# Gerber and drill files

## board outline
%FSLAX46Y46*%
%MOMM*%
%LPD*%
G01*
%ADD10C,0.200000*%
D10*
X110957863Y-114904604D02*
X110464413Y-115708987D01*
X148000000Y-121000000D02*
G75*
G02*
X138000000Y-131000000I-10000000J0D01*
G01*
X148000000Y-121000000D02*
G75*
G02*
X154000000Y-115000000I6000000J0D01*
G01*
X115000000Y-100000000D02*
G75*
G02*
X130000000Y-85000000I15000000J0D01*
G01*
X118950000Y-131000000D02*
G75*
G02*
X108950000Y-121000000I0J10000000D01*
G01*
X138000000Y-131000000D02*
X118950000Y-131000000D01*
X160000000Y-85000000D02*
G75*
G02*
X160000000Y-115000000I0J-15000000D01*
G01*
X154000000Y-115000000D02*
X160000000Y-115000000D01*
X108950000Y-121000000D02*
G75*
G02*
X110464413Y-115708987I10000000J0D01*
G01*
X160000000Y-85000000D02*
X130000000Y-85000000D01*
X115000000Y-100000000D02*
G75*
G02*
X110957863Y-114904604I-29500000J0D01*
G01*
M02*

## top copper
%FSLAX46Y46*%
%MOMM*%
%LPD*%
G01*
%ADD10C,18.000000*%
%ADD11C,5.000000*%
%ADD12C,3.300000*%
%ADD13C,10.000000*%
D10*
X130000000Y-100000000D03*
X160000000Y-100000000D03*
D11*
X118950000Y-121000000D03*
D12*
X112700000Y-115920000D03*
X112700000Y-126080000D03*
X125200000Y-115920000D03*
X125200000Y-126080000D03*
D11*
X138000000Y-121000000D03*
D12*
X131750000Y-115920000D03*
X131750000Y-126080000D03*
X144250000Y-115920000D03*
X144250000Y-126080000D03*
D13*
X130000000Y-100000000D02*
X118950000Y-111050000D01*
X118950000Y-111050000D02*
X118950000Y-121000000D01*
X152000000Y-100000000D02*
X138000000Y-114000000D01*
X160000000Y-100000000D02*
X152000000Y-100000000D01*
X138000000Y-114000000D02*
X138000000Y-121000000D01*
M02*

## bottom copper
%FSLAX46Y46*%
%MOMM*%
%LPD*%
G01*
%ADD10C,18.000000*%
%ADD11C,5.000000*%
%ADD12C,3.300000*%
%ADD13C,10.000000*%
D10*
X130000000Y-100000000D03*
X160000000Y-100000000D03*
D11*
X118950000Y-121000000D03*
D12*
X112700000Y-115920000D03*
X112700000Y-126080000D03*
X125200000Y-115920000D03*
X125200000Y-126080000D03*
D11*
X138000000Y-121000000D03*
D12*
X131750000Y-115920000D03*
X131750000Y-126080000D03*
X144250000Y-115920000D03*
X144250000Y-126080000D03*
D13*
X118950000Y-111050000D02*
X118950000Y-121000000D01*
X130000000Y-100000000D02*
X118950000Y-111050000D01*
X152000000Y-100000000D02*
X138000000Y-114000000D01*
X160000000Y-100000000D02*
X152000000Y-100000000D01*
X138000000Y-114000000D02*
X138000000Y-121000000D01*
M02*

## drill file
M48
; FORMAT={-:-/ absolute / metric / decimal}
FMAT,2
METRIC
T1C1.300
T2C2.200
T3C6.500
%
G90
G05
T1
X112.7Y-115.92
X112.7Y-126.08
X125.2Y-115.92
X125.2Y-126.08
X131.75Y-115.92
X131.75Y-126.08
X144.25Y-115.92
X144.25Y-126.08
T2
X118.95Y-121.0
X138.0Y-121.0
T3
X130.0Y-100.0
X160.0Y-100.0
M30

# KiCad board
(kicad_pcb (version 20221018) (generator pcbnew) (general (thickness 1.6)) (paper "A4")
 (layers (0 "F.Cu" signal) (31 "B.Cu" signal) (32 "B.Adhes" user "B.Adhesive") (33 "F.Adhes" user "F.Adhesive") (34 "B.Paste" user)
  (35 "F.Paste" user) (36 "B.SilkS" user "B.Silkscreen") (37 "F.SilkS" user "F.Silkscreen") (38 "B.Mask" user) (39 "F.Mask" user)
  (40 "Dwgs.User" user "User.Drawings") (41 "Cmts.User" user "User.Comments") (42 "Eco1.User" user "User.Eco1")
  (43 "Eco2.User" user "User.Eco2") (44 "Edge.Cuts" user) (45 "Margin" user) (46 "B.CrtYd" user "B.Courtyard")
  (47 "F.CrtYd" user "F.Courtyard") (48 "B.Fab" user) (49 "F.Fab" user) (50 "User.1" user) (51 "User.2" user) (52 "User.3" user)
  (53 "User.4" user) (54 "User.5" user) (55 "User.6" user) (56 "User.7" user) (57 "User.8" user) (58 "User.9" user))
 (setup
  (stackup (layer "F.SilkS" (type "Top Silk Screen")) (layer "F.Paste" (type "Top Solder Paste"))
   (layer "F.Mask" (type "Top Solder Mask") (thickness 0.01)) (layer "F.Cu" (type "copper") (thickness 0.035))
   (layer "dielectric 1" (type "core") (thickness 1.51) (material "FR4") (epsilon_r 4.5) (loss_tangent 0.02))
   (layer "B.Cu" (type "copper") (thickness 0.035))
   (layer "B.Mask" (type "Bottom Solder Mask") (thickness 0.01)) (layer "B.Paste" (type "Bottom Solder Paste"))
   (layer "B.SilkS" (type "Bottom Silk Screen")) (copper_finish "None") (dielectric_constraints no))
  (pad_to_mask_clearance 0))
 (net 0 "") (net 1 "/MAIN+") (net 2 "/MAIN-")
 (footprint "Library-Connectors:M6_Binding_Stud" (layer "F.Cu") (at 130 100)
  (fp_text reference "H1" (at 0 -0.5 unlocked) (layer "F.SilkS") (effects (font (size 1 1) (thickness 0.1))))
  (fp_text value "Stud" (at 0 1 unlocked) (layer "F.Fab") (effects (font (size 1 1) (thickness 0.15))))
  (pad "1" thru_hole circle (at 0 0) (size 18 18) (drill 6.5) (layers "*.Cu" "*.Mask") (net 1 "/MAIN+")))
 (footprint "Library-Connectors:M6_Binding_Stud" (layer "F.Cu") (at 160 100)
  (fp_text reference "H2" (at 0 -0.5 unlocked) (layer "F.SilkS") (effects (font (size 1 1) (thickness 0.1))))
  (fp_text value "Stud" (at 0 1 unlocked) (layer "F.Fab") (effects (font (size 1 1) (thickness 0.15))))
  (pad "1" thru_hole circle (at 0 0) (size 18 18) (drill 6.5) (layers "*.Cu" "*.Mask") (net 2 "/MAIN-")))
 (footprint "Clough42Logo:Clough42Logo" (layer "F.Cu") (at 145.5 87.5)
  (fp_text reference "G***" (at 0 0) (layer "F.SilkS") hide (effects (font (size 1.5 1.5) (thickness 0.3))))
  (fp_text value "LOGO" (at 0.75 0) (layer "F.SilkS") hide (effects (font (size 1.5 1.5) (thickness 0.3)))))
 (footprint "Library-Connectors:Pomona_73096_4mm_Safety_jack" (layer "F.Cu") (at 118.95 121)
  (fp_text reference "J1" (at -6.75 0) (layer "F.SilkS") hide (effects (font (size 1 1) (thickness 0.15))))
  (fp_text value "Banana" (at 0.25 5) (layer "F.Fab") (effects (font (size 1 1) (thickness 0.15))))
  (pad "1" thru_hole circle (at 0 0) (size 5 5) (drill 2.2) (layers "*.Cu" "*.Mask") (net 1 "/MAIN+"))
  (pad "2" thru_hole circle (at -6.25 -5.08) (size 3.3 3.3) (drill 1.3) (layers "*.Cu" "*.Mask"))
  (pad "2" thru_hole circle (at -6.25 5.08) (size 3.3 3.3) (drill 1.3) (layers "*.Cu" "*.Mask"))
  (pad "2" thru_hole circle (at 6.25 -5.08) (size 3.3 3.3) (drill 1.3) (layers "*.Cu" "*.Mask"))
  (pad "2" thru_hole circle (at 6.25 5.08) (size 3.3 3.3) (drill 1.3) (layers "*.Cu" "*.Mask")))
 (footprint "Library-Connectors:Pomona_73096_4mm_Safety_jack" (layer "F.Cu") (at 138 121)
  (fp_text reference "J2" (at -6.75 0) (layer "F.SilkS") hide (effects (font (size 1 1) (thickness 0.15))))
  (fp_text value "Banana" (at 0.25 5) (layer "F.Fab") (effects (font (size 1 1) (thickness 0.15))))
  (pad "1" thru_hole circle (at 0 0) (size 5 5) (drill 2.2) (layers "*.Cu" "*.Mask") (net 2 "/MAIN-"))
  (pad "2" thru_hole circle (at -6.25 -5.08) (size 3.3 3.3) (drill 1.3) (layers "*.Cu" "*.Mask"))
  (pad "2" thru_hole circle (at -6.25 5.08) (size 3.3 3.3) (drill 1.3) (layers "*.Cu" "*.Mask"))
  (pad "2" thru_hole circle (at 6.25 -5.08) (size 3.3 3.3) (drill 1.3) (layers "*.Cu" "*.Mask"))
  (pad "2" thru_hole circle (at 6.25 5.08) (size 3.3 3.3) (drill 1.3) (layers "*.Cu" "*.Mask")))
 (gr_line (start 110.957863 114.904604) (end 110.464413 115.708987) (stroke (width 0.2) (type default)) (layer "Edge.Cuts"))
 (gr_arc (start 148 121) (mid 145.071068 128.071067) (end 138 131) (stroke (width 0.2) (type default)) (layer "Edge.Cuts"))
 (gr_arc (start 148 121) (mid 149.757359 116.757359) (end 154 115) (stroke (width 0.2) (type default)) (layer "Edge.Cuts"))
 (gr_arc (start 115 100) (mid 119.393398 89.393399) (end 130 85) (stroke (width 0.2) (type default)) (layer "Edge.Cuts"))
 (gr_arc (start 118.95 131) (mid 111.878933 128.071068) (end 108.95 121) (stroke (width 0.2) (type default)) (layer "Edge.Cuts"))
 (gr_line (start 138 131) (end 118.95 131) (stroke (width 0.2) (type default)) (layer "Edge.Cuts"))
 (gr_arc (start 160 85) (mid 175 100) (end 160 115) (stroke (width 0.2) (type default)) (layer "Edge.Cuts"))
 (gr_line (start 154 115) (end 160 115) (stroke (width 0.2) (type default)) (layer "Edge.Cuts"))
 (gr_arc (start 108.95 121) (mid 109.336055 118.248261) (end 110.464413 115.708987) (stroke (width 0.2) (type default)) (layer "Edge.Cuts"))
 (gr_line (start 160 85) (end 130 85) (stroke (width 0.2) (type default)) (layer "Edge.Cuts"))
 (gr_arc (start 115 100) (mid 113.971538 107.721498) (end 110.957863 114.904604) (stroke (width 0.2) (type default)) (layer "Edge.Cuts"))
 (segment (start 130 100) (end 118.95 111.05) (width 10) (layer "F.Cu") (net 1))
 (segment (start 118.95 111.05) (end 118.95 121) (width 10) (layer "F.Cu") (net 1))
 (segment (start 118.95 111.05) (end 118.95 121) (width 10) (layer "B.Cu") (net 1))
 (segment (start 130 100) (end 118.95 111.05) (width 10) (layer "B.Cu") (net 1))
 (segment (start 152 100) (end 138 114) (width 10) (layer "F.Cu") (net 2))
 (segment (start 160 100) (end 152 100) (width 10) (layer "F.Cu") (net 2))
 (segment (start 138 114) (end 138 121) (width 10) (layer "F.Cu") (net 2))
 (segment (start 152 100) (end 138 114) (width 10) (layer "B.Cu") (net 2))
 (segment (start 160 100) (end 152 100) (width 10) (layer "B.Cu") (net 2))
 (segment (start 138 114) (end 138 121) (width 10) (layer "B.Cu") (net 2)))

